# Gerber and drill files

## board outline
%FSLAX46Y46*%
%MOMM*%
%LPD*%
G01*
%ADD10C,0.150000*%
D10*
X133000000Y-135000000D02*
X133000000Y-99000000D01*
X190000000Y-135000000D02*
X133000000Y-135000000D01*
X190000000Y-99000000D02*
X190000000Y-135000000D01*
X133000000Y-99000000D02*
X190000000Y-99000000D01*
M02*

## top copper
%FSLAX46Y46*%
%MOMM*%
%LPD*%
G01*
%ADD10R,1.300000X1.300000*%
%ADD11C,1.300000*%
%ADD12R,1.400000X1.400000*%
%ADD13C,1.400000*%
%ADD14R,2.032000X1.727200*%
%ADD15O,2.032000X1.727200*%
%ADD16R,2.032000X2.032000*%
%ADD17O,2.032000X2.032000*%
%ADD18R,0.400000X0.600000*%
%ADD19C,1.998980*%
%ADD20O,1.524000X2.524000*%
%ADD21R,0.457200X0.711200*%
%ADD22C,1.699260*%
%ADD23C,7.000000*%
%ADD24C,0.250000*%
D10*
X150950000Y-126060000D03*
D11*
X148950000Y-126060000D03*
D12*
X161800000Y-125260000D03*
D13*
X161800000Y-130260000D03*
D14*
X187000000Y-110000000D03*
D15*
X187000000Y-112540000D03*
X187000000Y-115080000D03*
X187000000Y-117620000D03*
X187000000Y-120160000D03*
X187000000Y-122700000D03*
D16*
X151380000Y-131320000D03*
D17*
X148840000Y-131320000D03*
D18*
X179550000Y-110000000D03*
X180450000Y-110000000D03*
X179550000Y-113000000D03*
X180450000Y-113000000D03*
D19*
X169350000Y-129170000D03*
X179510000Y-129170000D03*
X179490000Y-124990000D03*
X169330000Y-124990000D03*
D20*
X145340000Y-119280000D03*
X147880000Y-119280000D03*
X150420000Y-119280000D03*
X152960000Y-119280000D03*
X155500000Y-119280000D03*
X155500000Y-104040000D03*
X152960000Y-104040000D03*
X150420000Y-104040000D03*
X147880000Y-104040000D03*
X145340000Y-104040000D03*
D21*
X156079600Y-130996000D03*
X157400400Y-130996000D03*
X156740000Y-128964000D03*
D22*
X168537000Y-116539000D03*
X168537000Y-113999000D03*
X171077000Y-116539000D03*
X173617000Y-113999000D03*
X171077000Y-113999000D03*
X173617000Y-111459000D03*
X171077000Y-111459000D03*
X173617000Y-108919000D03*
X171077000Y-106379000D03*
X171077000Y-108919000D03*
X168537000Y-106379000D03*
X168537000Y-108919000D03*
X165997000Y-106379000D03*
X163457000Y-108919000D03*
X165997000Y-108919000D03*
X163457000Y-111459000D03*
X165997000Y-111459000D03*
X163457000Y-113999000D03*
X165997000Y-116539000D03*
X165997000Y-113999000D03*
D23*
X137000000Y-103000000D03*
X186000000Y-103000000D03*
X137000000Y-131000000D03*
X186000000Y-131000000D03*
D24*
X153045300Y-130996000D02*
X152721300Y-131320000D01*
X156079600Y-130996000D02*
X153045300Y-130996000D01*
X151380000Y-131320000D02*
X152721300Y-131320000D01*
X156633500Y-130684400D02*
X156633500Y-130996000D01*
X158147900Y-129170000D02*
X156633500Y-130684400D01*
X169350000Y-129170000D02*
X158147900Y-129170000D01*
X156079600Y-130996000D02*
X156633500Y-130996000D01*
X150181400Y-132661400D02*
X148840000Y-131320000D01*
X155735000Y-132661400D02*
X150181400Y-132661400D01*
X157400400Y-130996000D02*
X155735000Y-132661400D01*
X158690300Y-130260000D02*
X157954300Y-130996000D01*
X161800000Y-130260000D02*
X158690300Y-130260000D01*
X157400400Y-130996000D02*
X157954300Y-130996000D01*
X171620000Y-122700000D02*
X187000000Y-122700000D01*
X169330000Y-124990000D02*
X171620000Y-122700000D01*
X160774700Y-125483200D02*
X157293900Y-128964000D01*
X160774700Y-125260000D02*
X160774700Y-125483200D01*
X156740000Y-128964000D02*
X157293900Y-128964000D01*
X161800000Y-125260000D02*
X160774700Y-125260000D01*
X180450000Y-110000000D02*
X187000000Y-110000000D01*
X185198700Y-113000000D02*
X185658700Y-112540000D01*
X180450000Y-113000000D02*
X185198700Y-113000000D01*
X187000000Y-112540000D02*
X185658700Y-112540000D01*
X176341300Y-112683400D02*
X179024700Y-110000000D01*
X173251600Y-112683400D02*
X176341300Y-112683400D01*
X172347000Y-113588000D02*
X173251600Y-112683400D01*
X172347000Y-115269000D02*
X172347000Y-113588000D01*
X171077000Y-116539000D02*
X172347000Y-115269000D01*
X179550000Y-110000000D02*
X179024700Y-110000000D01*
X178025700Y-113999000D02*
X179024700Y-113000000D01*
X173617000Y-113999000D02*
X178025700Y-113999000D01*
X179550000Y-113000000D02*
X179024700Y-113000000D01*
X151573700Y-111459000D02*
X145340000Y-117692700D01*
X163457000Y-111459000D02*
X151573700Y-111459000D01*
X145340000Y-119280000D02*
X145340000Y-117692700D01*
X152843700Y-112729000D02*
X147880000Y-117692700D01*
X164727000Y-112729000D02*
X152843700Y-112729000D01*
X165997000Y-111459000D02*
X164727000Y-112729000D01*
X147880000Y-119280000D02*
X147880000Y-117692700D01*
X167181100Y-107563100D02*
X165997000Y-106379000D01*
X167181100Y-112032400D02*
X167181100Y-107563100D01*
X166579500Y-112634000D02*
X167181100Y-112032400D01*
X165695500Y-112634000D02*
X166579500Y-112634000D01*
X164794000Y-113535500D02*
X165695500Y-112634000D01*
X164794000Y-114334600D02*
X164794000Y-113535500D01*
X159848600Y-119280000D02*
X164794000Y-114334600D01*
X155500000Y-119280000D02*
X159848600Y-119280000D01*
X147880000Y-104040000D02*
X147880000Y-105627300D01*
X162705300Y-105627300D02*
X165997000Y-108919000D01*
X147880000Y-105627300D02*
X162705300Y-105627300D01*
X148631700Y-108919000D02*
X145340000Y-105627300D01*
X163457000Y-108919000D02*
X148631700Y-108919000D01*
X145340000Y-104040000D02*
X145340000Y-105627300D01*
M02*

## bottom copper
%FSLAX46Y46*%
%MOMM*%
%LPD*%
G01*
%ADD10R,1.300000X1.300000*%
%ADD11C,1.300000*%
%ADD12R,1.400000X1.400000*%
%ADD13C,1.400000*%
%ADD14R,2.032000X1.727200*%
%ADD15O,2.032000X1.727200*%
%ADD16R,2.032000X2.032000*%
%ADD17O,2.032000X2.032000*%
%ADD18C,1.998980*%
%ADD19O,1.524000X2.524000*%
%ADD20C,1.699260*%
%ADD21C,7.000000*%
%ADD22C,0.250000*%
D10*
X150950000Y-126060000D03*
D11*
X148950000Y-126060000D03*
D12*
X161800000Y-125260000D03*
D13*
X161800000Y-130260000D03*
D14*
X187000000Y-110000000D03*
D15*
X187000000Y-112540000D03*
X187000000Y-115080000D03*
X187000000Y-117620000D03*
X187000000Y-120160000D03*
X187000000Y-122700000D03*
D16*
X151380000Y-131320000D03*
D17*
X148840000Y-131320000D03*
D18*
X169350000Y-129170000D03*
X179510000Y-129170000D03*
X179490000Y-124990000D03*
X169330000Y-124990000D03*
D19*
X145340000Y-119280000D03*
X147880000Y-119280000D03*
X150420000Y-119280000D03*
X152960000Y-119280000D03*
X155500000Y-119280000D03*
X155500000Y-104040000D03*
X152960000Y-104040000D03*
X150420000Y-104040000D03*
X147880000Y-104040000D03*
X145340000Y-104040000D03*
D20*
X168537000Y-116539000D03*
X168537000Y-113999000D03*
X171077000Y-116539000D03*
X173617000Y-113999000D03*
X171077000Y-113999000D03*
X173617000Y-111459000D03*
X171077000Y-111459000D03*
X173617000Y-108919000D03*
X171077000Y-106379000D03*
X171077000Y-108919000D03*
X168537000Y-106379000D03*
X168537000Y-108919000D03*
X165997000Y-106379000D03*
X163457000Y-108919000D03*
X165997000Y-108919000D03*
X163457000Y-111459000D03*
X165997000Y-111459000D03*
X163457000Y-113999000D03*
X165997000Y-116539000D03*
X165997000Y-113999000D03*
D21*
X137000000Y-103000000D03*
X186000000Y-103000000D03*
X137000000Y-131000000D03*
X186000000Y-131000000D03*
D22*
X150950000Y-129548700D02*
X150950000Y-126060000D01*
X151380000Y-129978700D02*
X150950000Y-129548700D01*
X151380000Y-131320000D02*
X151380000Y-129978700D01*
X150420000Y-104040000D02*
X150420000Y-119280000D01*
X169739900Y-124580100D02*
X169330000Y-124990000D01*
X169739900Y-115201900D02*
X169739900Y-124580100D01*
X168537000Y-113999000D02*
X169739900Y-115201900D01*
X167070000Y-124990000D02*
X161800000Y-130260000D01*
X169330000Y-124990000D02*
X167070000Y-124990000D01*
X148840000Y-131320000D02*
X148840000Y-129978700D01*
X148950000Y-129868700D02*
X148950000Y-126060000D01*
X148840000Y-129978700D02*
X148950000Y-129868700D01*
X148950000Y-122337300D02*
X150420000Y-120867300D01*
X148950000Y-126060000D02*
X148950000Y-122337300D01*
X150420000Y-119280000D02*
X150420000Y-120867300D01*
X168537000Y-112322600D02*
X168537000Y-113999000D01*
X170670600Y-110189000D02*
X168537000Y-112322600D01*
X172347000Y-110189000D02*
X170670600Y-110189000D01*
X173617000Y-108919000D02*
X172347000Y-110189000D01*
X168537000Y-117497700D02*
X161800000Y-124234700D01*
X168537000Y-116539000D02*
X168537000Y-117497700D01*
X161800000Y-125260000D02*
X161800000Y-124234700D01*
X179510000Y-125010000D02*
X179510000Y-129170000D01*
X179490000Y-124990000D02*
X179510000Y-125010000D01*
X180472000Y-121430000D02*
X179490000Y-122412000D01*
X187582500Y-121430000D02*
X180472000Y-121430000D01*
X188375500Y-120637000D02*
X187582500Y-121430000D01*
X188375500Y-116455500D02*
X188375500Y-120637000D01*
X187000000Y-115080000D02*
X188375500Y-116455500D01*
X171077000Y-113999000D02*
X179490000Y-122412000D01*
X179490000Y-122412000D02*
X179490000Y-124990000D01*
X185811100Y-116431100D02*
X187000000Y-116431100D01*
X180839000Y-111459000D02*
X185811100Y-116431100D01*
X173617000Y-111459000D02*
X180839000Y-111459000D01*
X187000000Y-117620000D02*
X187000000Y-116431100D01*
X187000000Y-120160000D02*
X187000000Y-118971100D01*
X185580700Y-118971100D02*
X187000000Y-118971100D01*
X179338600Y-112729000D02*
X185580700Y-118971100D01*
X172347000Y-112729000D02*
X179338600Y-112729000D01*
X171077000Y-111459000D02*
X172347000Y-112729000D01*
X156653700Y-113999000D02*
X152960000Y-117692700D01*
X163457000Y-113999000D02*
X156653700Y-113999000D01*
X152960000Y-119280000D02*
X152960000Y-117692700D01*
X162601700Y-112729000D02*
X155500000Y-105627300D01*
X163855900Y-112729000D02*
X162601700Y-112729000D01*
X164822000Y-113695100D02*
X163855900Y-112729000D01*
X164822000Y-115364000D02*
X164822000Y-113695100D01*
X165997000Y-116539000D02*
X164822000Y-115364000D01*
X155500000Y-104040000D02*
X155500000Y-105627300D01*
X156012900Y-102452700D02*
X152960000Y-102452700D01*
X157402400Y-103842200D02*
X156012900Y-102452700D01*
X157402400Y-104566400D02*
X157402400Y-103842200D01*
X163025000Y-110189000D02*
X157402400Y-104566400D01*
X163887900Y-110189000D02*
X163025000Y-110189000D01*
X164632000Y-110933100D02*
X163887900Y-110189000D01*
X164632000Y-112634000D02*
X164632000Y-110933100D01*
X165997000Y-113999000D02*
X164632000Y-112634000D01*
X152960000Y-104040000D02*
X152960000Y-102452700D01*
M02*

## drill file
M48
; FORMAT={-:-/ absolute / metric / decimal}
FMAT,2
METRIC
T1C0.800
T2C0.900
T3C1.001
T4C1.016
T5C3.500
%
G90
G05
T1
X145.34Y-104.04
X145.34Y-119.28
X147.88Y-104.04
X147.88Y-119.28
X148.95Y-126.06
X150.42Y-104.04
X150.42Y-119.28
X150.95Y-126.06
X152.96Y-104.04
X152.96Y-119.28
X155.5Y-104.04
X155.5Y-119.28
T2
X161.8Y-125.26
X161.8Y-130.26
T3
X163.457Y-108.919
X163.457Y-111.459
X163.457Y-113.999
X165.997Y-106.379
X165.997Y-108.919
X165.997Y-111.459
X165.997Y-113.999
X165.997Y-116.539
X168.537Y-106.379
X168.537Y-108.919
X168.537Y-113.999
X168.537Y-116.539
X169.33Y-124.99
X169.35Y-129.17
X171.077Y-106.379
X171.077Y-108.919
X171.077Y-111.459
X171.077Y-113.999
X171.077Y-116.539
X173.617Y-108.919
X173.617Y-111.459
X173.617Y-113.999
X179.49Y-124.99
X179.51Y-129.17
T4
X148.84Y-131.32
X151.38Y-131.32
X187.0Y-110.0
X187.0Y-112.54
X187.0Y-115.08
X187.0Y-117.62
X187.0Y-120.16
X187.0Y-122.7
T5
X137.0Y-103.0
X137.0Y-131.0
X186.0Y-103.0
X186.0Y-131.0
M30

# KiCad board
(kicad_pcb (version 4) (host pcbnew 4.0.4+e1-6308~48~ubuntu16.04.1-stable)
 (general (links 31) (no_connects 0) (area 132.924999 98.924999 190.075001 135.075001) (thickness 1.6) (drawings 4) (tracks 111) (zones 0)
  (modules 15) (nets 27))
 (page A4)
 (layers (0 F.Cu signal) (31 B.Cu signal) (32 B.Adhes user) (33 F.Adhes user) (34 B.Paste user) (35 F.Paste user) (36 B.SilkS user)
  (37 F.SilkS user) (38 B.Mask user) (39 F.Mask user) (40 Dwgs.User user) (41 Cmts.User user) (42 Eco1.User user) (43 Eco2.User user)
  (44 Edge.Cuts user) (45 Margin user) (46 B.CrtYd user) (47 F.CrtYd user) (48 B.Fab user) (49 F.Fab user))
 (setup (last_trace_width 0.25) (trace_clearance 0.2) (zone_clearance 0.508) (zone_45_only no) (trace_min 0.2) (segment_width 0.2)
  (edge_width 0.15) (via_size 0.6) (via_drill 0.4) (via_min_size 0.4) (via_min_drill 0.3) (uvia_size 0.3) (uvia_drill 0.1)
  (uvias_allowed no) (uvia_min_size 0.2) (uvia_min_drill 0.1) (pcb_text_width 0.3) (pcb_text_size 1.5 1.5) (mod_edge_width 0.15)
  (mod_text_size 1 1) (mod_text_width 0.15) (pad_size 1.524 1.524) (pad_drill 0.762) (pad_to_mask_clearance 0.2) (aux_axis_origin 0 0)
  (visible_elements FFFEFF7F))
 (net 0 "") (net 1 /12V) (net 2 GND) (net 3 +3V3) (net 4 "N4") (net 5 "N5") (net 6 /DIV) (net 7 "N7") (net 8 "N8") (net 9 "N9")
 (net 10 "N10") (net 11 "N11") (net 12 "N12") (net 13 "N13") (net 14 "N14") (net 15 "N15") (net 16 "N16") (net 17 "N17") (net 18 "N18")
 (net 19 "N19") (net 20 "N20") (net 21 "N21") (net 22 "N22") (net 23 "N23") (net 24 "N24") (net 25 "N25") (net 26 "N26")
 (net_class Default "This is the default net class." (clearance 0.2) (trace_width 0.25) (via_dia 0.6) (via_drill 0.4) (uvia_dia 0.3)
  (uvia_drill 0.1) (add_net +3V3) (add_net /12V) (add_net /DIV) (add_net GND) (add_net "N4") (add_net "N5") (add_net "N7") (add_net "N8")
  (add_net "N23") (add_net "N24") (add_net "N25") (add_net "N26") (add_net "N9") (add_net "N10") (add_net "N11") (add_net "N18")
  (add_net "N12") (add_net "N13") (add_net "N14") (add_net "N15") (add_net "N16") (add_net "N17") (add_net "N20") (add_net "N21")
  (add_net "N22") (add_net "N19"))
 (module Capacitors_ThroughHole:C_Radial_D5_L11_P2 (layer F.Cu) (at 150.95 126.06 180)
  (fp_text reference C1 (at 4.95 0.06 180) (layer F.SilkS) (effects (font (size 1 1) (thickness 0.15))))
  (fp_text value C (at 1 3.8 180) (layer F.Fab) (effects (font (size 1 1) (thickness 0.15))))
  (pad 1 thru_hole rect (at 0 0 180) (size 1.3 1.3) (drill 0.8) (layers *.Cu *.Mask F.SilkS) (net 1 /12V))
  (pad 2 thru_hole circle (at 2 0 180) (size 1.3 1.3) (drill 0.8) (layers *.Cu *.Mask F.SilkS) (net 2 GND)))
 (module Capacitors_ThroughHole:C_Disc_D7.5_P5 (layer F.Cu) (at 161.8 125.26 270)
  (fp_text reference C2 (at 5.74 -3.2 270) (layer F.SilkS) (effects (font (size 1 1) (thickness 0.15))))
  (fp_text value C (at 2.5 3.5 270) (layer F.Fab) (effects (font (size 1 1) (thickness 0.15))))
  (pad 1 thru_hole rect (at 0 0 270) (size 1.4 1.4) (drill 0.9) (layers *.Cu *.Mask F.SilkS) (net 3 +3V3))
  (pad 2 thru_hole circle (at 5 0 270) (size 1.4 1.4) (drill 0.9) (layers *.Cu *.Mask F.SilkS) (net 2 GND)))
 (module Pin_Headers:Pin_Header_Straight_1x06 (layer F.Cu) (at 187 110)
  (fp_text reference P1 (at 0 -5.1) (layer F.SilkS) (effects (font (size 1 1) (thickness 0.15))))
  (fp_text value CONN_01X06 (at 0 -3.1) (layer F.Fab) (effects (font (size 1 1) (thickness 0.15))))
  (pad 1 thru_hole rect (at 0 0) (size 2.032 1.7272) (drill 1.016) (layers *.Cu *.Mask F.SilkS) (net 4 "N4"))
  (pad 2 thru_hole oval (at 0 2.54) (size 2.032 1.7272) (drill 1.016) (layers *.Cu *.Mask F.SilkS) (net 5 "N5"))
  (pad 3 thru_hole oval (at 0 5.08) (size 2.032 1.7272) (drill 1.016) (layers *.Cu *.Mask F.SilkS) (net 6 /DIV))
  (pad 4 thru_hole oval (at 0 7.62) (size 2.032 1.7272) (drill 1.016) (layers *.Cu *.Mask F.SilkS) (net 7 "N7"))
  (pad 5 thru_hole oval (at 0 10.16) (size 2.032 1.7272) (drill 1.016) (layers *.Cu *.Mask F.SilkS) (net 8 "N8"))
  (pad 6 thru_hole oval (at 0 12.7) (size 2.032 1.7272) (drill 1.016) (layers *.Cu *.Mask F.SilkS) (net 2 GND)))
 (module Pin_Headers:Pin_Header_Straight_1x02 (layer F.Cu) (at 151.38 131.32 270)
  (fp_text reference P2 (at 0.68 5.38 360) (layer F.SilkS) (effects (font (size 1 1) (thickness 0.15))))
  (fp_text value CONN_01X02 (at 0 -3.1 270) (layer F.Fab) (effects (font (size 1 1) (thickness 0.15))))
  (pad 1 thru_hole rect (at 0 0 270) (size 2.032 2.032) (drill 1.016) (layers *.Cu *.Mask F.SilkS) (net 1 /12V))
  (pad 2 thru_hole oval (at 0 2.54 270) (size 2.032 2.032) (drill 1.016) (layers *.Cu *.Mask F.SilkS) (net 2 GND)))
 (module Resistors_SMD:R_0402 (layer F.Cu) (at 180 110)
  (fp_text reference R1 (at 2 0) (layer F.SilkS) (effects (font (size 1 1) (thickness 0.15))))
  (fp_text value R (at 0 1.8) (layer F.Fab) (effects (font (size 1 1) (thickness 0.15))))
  (pad 1 smd rect (at -0.45 0) (size 0.4 0.6) (layers F.Cu F.Paste F.Mask) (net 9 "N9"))
  (pad 2 smd rect (at 0.45 0) (size 0.4 0.6) (layers F.Cu F.Paste F.Mask) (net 4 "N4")))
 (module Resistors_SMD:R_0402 (layer F.Cu) (at 180 113)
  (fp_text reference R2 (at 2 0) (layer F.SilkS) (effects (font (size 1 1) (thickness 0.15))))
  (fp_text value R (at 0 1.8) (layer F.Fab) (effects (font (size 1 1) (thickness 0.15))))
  (pad 1 smd rect (at -0.45 0) (size 0.4 0.6) (layers F.Cu F.Paste F.Mask) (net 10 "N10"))
  (pad 2 smd rect (at 0.45 0) (size 0.4 0.6) (layers F.Cu F.Paste F.Mask) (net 5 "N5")))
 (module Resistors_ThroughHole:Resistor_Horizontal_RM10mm (layer F.Cu) (at 169.35 129.17)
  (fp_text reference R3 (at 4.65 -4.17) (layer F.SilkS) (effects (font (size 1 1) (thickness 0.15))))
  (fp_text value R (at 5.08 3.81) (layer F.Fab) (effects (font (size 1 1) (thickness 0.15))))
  (pad 1 thru_hole circle (at 0 0) (size 1.99898 1.99898) (drill 1.00076) (layers *.Cu *.SilkS *.Mask) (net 1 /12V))
  (pad 2 thru_hole circle (at 10.16 0) (size 1.99898 1.99898) (drill 1.00076) (layers *.Cu *.SilkS *.Mask) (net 6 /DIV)))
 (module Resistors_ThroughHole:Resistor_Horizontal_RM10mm (layer F.Cu) (at 179.49 124.99 180)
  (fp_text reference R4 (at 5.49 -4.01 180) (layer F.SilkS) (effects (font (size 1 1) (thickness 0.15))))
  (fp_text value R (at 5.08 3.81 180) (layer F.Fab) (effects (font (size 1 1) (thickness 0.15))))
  (pad 1 thru_hole circle (at 0 0 180) (size 1.99898 1.99898) (drill 1.00076) (layers *.Cu *.SilkS *.Mask) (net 6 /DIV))
  (pad 2 thru_hole circle (at 10.16 0 180) (size 1.99898 1.99898) (drill 1.00076) (layers *.Cu *.SilkS *.Mask) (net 2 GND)))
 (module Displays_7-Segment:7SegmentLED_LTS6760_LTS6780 (layer F.Cu) (at 150.42 111.66)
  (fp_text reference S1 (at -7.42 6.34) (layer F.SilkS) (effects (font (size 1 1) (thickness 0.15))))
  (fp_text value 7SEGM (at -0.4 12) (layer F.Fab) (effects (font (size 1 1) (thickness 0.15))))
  (pad 1 thru_hole oval (at -5.08 7.62) (size 1.524 2.524) (drill 0.8) (layers *.Cu *.Mask F.SilkS) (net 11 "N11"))
  (pad 2 thru_hole oval (at -2.54 7.62) (size 1.524 2.524) (drill 0.8) (layers *.Cu *.Mask F.SilkS) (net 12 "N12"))
  (pad 3 thru_hole oval (at 0 7.62) (size 1.524 2.524) (drill 0.8) (layers *.Cu *.Mask F.SilkS) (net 2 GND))
  (pad 4 thru_hole oval (at 2.54 7.62) (size 1.524 2.524) (drill 0.8) (layers *.Cu *.Mask F.SilkS) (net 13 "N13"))
  (pad 5 thru_hole oval (at 5.08 7.62) (size 1.524 2.524) (drill 0.8) (layers *.Cu *.Mask F.SilkS) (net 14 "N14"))
  (pad 6 thru_hole oval (at 5.08 -7.62) (size 1.524 2.524) (drill 0.8) (layers *.Cu *.Mask F.SilkS) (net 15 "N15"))
  (pad 7 thru_hole oval (at 2.54 -7.62) (size 1.524 2.524) (drill 0.8) (layers *.Cu *.Mask F.SilkS) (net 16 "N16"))
  (pad 8 thru_hole oval (at 0 -7.62) (size 1.524 2.524) (drill 0.8) (layers *.Cu *.Mask F.SilkS) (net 2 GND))
  (pad 9 thru_hole oval (at -2.54 -7.62) (size 1.524 2.524) (drill 0.8) (layers *.Cu *.Mask F.SilkS) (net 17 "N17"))
  (pad 10 thru_hole oval (at -5.08 -7.62) (size 1.524 2.524) (drill 0.8) (layers *.Cu *.Mask F.SilkS) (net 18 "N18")))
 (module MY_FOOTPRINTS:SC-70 (layer F.Cu) (at 156.74 129.98)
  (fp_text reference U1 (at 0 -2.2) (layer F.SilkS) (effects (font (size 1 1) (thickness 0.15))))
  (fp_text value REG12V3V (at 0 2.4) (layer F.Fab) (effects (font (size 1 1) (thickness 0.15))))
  (pad 1 smd rect (at -0.6604 1.016) (size 0.4572 0.7112) (layers F.Cu F.Paste F.Mask) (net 1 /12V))
  (pad 2 smd rect (at 0.6604 1.016) (size 0.4572 0.7112) (layers F.Cu F.Paste F.Mask) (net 2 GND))
  (pad 3 smd rect (at 0 -1.016) (size 0.4572 0.7112) (layers F.Cu F.Paste F.Mask) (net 3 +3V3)))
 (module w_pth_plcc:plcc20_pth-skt (layer F.Cu) (at 168.537 111.459)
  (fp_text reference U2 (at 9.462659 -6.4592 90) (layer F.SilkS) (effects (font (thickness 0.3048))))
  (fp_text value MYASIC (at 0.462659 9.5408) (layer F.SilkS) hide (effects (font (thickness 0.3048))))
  (pad 1 thru_hole circle (at 0 5.08) (size 1.69926 1.69926) (drill 1.00076) (layers *.Cu *.Mask F.SilkS) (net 3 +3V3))
  (pad 2 thru_hole circle (at 0 2.54) (size 1.69926 1.69926) (drill 1.00076) (layers *.Cu *.Mask F.SilkS) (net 2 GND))
  (pad 3 thru_hole circle (at 2.54 5.08) (size 1.69926 1.69926) (drill 1.00076) (layers *.Cu *.Mask F.SilkS) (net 9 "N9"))
  (pad 4 thru_hole circle (at 5.08 2.54) (size 1.69926 1.69926) (drill 1.00076) (layers *.Cu *.Mask F.SilkS) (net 10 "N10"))
  (pad 5 thru_hole circle (at 2.54 2.54) (size 1.69926 1.69926) (drill 1.00076) (layers *.Cu *.Mask F.SilkS) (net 6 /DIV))
  (pad 6 thru_hole circle (at 5.08 0) (size 1.69926 1.69926) (drill 1.00076) (layers *.Cu *.Mask F.SilkS) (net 7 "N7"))
  (pad 7 thru_hole circle (at 2.54 0) (size 1.69926 1.69926) (drill 1.00076) (layers *.Cu *.Mask F.SilkS) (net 8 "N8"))
  (pad 8 thru_hole circle (at 5.08 -2.54) (size 1.69926 1.69926) (drill 1.00076) (layers *.Cu *.Mask F.SilkS) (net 2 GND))
  (pad 9 thru_hole circle (at 2.54 -5.08) (size 1.69926 1.69926) (drill 1.00076) (layers *.Cu *.Mask F.SilkS) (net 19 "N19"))
  (pad 10 thru_hole circle (at 2.54 -2.54) (size 1.69926 1.69926) (drill 1.00076) (layers *.Cu *.Mask F.SilkS) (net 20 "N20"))
  (pad 11 thru_hole circle (at 0 -5.08) (size 1.69926 1.69926) (drill 1.00076) (layers *.Cu *.Mask F.SilkS) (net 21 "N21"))
  (pad 12 thru_hole circle (at 0 -2.54) (size 1.69926 1.69926) (drill 1.00076) (layers *.Cu *.Mask F.SilkS) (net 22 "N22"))
  (pad 13 thru_hole circle (at -2.54 -5.08) (size 1.69926 1.69926) (drill 1.00076) (layers *.Cu *.Mask F.SilkS) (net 14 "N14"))
  (pad 14 thru_hole circle (at -5.08 -2.54) (size 1.69926 1.69926) (drill 1.00076) (layers *.Cu *.Mask F.SilkS) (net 18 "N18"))
  (pad 15 thru_hole circle (at -2.54 -2.54) (size 1.69926 1.69926) (drill 1.00076) (layers *.Cu *.Mask F.SilkS) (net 17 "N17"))
  (pad 16 thru_hole circle (at -5.08 0) (size 1.69926 1.69926) (drill 1.00076) (layers *.Cu *.Mask F.SilkS) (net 11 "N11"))
  (pad 17 thru_hole circle (at -2.54 0) (size 1.69926 1.69926) (drill 1.00076) (layers *.Cu *.Mask F.SilkS) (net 12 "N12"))
  (pad 18 thru_hole circle (at -5.08 2.54) (size 1.69926 1.69926) (drill 1.00076) (layers *.Cu *.Mask F.SilkS) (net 13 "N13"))
  (pad 19 thru_hole circle (at -2.54 5.08) (size 1.69926 1.69926) (drill 1.00076) (layers *.Cu *.Mask F.SilkS) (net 15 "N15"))
  (pad 20 thru_hole circle (at -2.54 2.54) (size 1.69926 1.69926) (drill 1.00076) (layers *.Cu *.Mask F.SilkS) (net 16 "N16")))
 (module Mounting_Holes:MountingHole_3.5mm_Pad (layer F.Cu) (at 137 103)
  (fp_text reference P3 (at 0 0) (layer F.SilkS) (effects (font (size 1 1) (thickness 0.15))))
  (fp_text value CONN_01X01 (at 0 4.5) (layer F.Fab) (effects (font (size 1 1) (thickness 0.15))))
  (pad 1 thru_hole circle (at 0 0) (size 7 7) (drill 3.5) (layers *.Cu *.Mask F.SilkS) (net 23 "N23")))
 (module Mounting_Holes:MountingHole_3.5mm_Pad (layer F.Cu) (at 186 103)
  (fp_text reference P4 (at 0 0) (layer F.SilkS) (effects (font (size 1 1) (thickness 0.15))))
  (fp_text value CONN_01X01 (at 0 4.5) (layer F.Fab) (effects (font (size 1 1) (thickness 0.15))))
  (pad 1 thru_hole circle (at 0 0) (size 7 7) (drill 3.5) (layers *.Cu *.Mask F.SilkS) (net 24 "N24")))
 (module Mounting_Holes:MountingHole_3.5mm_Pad (layer F.Cu) (at 137 131)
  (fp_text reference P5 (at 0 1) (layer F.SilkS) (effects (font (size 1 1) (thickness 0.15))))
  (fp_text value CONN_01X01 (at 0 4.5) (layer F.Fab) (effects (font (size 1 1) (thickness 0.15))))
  (pad 1 thru_hole circle (at 0 0) (size 7 7) (drill 3.5) (layers *.Cu *.Mask F.SilkS) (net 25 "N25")))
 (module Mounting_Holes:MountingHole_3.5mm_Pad (layer F.Cu) (at 186 131)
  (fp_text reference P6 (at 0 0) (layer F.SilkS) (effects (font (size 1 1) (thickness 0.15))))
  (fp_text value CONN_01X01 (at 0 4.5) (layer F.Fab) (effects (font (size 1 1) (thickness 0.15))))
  (pad 1 thru_hole circle (at 0 0) (size 7 7) (drill 3.5) (layers *.Cu *.Mask F.SilkS) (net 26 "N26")))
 (gr_line (start 133 135) (end 133 99) (angle 90) (layer Edge.Cuts) (width 0.15))
 (gr_line (start 190 135) (end 133 135) (angle 90) (layer Edge.Cuts) (width 0.15))
 (gr_line (start 190 99) (end 190 135) (angle 90) (layer Edge.Cuts) (width 0.15))
 (gr_line (start 133 99) (end 190 99) (angle 90) (layer Edge.Cuts) (width 0.15))
 (segment (start 153.0453 130.996) (end 152.7213 131.32) (width 0.25) (layer F.Cu) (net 1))
 (segment (start 156.0796 130.996) (end 153.0453 130.996) (width 0.25) (layer F.Cu) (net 1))
 (segment (start 151.38 131.32) (end 152.7213 131.32) (width 0.25) (layer F.Cu) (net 1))
 (segment (start 156.6335 130.6844) (end 156.6335 130.996) (width 0.25) (layer F.Cu) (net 1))
 (segment (start 158.1479 129.17) (end 156.6335 130.6844) (width 0.25) (layer F.Cu) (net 1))
 (segment (start 169.35 129.17) (end 158.1479 129.17) (width 0.25) (layer F.Cu) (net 1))
 (segment (start 156.0796 130.996) (end 156.6335 130.996) (width 0.25) (layer F.Cu) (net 1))
 (segment (start 150.95 129.5487) (end 150.95 126.06) (width 0.25) (layer B.Cu) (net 1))
 (segment (start 151.38 129.9787) (end 150.95 129.5487) (width 0.25) (layer B.Cu) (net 1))
 (segment (start 151.38 131.32) (end 151.38 129.9787) (width 0.25) (layer B.Cu) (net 1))
 (segment (start 150.42 104.04) (end 150.42 119.28) (width 0.25) (layer B.Cu) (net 2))
 (segment (start 169.7399 124.5801) (end 169.33 124.99) (width 0.25) (layer B.Cu) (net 2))
 (segment (start 169.7399 115.2019) (end 169.7399 124.5801) (width 0.25) (layer B.Cu) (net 2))
 (segment (start 168.537 113.999) (end 169.7399 115.2019) (width 0.25) (layer B.Cu) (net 2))
 (segment (start 167.07 124.99) (end 161.8 130.26) (width 0.25) (layer B.Cu) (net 2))
 (segment (start 169.33 124.99) (end 167.07 124.99) (width 0.25) (layer B.Cu) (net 2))
 (segment (start 148.84 131.32) (end 148.84 129.9787) (width 0.25) (layer B.Cu) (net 2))
 (segment (start 150.1814 132.6614) (end 148.84 131.32) (width 0.25) (layer F.Cu) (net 2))
 (segment (start 155.735 132.6614) (end 150.1814 132.6614) (width 0.25) (layer F.Cu) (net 2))
 (segment (start 157.4004 130.996) (end 155.735 132.6614) (width 0.25) (layer F.Cu) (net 2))
 (segment (start 148.95 129.8687) (end 148.95 126.06) (width 0.25) (layer B.Cu) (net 2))
 (segment (start 148.84 129.9787) (end 148.95 129.8687) (width 0.25) (layer B.Cu) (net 2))
 (segment (start 148.95 122.3373) (end 150.42 120.8673) (width 0.25) (layer B.Cu) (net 2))
 (segment (start 148.95 126.06) (end 148.95 122.3373) (width 0.25) (layer B.Cu) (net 2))
 (segment (start 150.42 119.28) (end 150.42 120.8673) (width 0.25) (layer B.Cu) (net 2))
 (segment (start 158.6903 130.26) (end 157.9543 130.996) (width 0.25) (layer F.Cu) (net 2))
 (segment (start 161.8 130.26) (end 158.6903 130.26) (width 0.25) (layer F.Cu) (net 2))
 (segment (start 157.4004 130.996) (end 157.9543 130.996) (width 0.25) (layer F.Cu) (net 2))
 (segment (start 168.537 112.3226) (end 168.537 113.999) (width 0.25) (layer B.Cu) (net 2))
 (segment (start 170.6706 110.189) (end 168.537 112.3226) (width 0.25) (layer B.Cu) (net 2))
 (segment (start 172.347 110.189) (end 170.6706 110.189) (width 0.25) (layer B.Cu) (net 2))
 (segment (start 173.617 108.919) (end 172.347 110.189) (width 0.25) (layer B.Cu) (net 2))
 (segment (start 171.62 122.7) (end 187 122.7) (width 0.25) (layer F.Cu) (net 2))
 (segment (start 169.33 124.99) (end 171.62 122.7) (width 0.25) (layer F.Cu) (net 2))
 (segment (start 168.537 117.4977) (end 161.8 124.2347) (width 0.25) (layer B.Cu) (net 3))
 (segment (start 168.537 116.539) (end 168.537 117.4977) (width 0.25) (layer B.Cu) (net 3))
 (segment (start 161.8 125.26) (end 161.8 124.2347) (width 0.25) (layer B.Cu) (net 3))
 (segment (start 160.7747 125.4832) (end 157.2939 128.964) (width 0.25) (layer F.Cu) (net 3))
 (segment (start 160.7747 125.26) (end 160.7747 125.4832) (width 0.25) (layer F.Cu) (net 3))
 (segment (start 156.74 128.964) (end 157.2939 128.964) (width 0.25) (layer F.Cu) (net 3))
 (segment (start 161.8 125.26) (end 160.7747 125.26) (width 0.25) (layer F.Cu) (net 3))
 (segment (start 180.45 110) (end 187 110) (width 0.25) (layer F.Cu) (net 4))
 (segment (start 185.1987 113) (end 185.6587 112.54) (width 0.25) (layer F.Cu) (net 5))
 (segment (start 180.45 113) (end 185.1987 113) (width 0.25) (layer F.Cu) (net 5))
 (segment (start 187 112.54) (end 185.6587 112.54) (width 0.25) (layer F.Cu) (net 5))
 (segment (start 179.51 125.01) (end 179.51 129.17) (width 0.25) (layer B.Cu) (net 6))
 (segment (start 179.49 124.99) (end 179.51 125.01) (width 0.25) (layer B.Cu) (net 6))
 (segment (start 180.472 121.43) (end 179.49 122.412) (width 0.25) (layer B.Cu) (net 6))
 (segment (start 187.5825 121.43) (end 180.472 121.43) (width 0.25) (layer B.Cu) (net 6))
 (segment (start 188.3755 120.637) (end 187.5825 121.43) (width 0.25) (layer B.Cu) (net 6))
 (segment (start 188.3755 116.4555) (end 188.3755 120.637) (width 0.25) (layer B.Cu) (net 6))
 (segment (start 187 115.08) (end 188.3755 116.4555) (width 0.25) (layer B.Cu) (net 6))
 (segment (start 171.077 113.999) (end 179.49 122.412) (width 0.25) (layer B.Cu) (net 6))
 (segment (start 179.49 122.412) (end 179.49 124.99) (width 0.25) (layer B.Cu) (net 6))
 (segment (start 185.8111 116.4311) (end 187 116.4311) (width 0.25) (layer B.Cu) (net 7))
 (segment (start 180.839 111.459) (end 185.8111 116.4311) (width 0.25) (layer B.Cu) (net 7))
 (segment (start 173.617 111.459) (end 180.839 111.459) (width 0.25) (layer B.Cu) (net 7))
 (segment (start 187 117.62) (end 187 116.4311) (width 0.25) (layer B.Cu) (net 7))
 (segment (start 187 120.16) (end 187 118.9711) (width 0.25) (layer B.Cu) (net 8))
 (segment (start 185.5807 118.9711) (end 187 118.9711) (width 0.25) (layer B.Cu) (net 8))
 (segment (start 179.3386 112.729) (end 185.5807 118.9711) (width 0.25) (layer B.Cu) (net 8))
 (segment (start 172.347 112.729) (end 179.3386 112.729) (width 0.25) (layer B.Cu) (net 8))
 (segment (start 171.077 111.459) (end 172.347 112.729) (width 0.25) (layer B.Cu) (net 8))
 (segment (start 176.3413 112.6834) (end 179.0247 110) (width 0.25) (layer F.Cu) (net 9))
 (segment (start 173.2516 112.6834) (end 176.3413 112.6834) (width 0.25) (layer F.Cu) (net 9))
 (segment (start 172.347 113.588) (end 173.2516 112.6834) (width 0.25) (layer F.Cu) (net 9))
 (segment (start 172.347 115.269) (end 172.347 113.588) (width 0.25) (layer F.Cu) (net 9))
 (segment (start 171.077 116.539) (end 172.347 115.269) (width 0.25) (layer F.Cu) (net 9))
 (segment (start 179.55 110) (end 179.0247 110) (width 0.25) (layer F.Cu) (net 9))
 (segment (start 178.0257 113.999) (end 179.0247 113) (width 0.25) (layer F.Cu) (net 10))
 (segment (start 173.617 113.999) (end 178.0257 113.999) (width 0.25) (layer F.Cu) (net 10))
 (segment (start 179.55 113) (end 179.0247 113) (width 0.25) (layer F.Cu) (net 10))
 (segment (start 151.5737 111.459) (end 145.34 117.6927) (width 0.25) (layer F.Cu) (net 11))
 (segment (start 163.457 111.459) (end 151.5737 111.459) (width 0.25) (layer F.Cu) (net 11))
 (segment (start 145.34 119.28) (end 145.34 117.6927) (width 0.25) (layer F.Cu) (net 11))
 (segment (start 152.8437 112.729) (end 147.88 117.6927) (width 0.25) (layer F.Cu) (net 12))
 (segment (start 164.727 112.729) (end 152.8437 112.729) (width 0.25) (layer F.Cu) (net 12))
 (segment (start 165.997 111.459) (end 164.727 112.729) (width 0.25) (layer F.Cu) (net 12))
 (segment (start 147.88 119.28) (end 147.88 117.6927) (width 0.25) (layer F.Cu) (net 12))
 (segment (start 156.6537 113.999) (end 152.96 117.6927) (width 0.25) (layer B.Cu) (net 13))
 (segment (start 163.457 113.999) (end 156.6537 113.999) (width 0.25) (layer B.Cu) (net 13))
 (segment (start 152.96 119.28) (end 152.96 117.6927) (width 0.25) (layer B.Cu) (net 13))
 (segment (start 167.1811 107.5631) (end 165.997 106.379) (width 0.25) (layer F.Cu) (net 14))
 (segment (start 167.1811 112.0324) (end 167.1811 107.5631) (width 0.25) (layer F.Cu) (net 14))
 (segment (start 166.5795 112.634) (end 167.1811 112.0324) (width 0.25) (layer F.Cu) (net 14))
 (segment (start 165.6955 112.634) (end 166.5795 112.634) (width 0.25) (layer F.Cu) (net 14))
 (segment (start 164.794 113.5355) (end 165.6955 112.634) (width 0.25) (layer F.Cu) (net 14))
 (segment (start 164.794 114.3346) (end 164.794 113.5355) (width 0.25) (layer F.Cu) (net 14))
 (segment (start 159.8486 119.28) (end 164.794 114.3346) (width 0.25) (layer F.Cu) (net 14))
 (segment (start 155.5 119.28) (end 159.8486 119.28) (width 0.25) (layer F.Cu) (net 14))
 (segment (start 162.6017 112.729) (end 155.5 105.6273) (width 0.25) (layer B.Cu) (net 15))
 (segment (start 163.8559 112.729) (end 162.6017 112.729) (width 0.25) (layer B.Cu) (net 15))
 (segment (start 164.822 113.6951) (end 163.8559 112.729) (width 0.25) (layer B.Cu) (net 15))
 (segment (start 164.822 115.364) (end 164.822 113.6951) (width 0.25) (layer B.Cu) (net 15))
 (segment (start 165.997 116.539) (end 164.822 115.364) (width 0.25) (layer B.Cu) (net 15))
 (segment (start 155.5 104.04) (end 155.5 105.6273) (width 0.25) (layer B.Cu) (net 15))
 (segment (start 156.0129 102.4527) (end 152.96 102.4527) (width 0.25) (layer B.Cu) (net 16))
 (segment (start 157.4024 103.8422) (end 156.0129 102.4527) (width 0.25) (layer B.Cu) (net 16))
 (segment (start 157.4024 104.5664) (end 157.4024 103.8422) (width 0.25) (layer B.Cu) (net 16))
 (segment (start 163.025 110.189) (end 157.4024 104.5664) (width 0.25) (layer B.Cu) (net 16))
 (segment (start 163.8879 110.189) (end 163.025 110.189) (width 0.25) (layer B.Cu) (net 16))
 (segment (start 164.632 110.9331) (end 163.8879 110.189) (width 0.25) (layer B.Cu) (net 16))
 (segment (start 164.632 112.634) (end 164.632 110.9331) (width 0.25) (layer B.Cu) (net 16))
 (segment (start 165.997 113.999) (end 164.632 112.634) (width 0.25) (layer B.Cu) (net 16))
 (segment (start 152.96 104.04) (end 152.96 102.4527) (width 0.25) (layer B.Cu) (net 16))
 (segment (start 147.88 104.04) (end 147.88 105.6273) (width 0.25) (layer F.Cu) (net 17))
 (segment (start 162.7053 105.6273) (end 165.997 108.919) (width 0.25) (layer F.Cu) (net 17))
 (segment (start 147.88 105.6273) (end 162.7053 105.6273) (width 0.25) (layer F.Cu) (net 17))
 (segment (start 148.6317 108.919) (end 145.34 105.6273) (width 0.25) (layer F.Cu) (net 18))
 (segment (start 163.457 108.919) (end 148.6317 108.919) (width 0.25) (layer F.Cu) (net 18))
 (segment (start 145.34 104.04) (end 145.34 105.6273) (width 0.25) (layer F.Cu) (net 18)))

